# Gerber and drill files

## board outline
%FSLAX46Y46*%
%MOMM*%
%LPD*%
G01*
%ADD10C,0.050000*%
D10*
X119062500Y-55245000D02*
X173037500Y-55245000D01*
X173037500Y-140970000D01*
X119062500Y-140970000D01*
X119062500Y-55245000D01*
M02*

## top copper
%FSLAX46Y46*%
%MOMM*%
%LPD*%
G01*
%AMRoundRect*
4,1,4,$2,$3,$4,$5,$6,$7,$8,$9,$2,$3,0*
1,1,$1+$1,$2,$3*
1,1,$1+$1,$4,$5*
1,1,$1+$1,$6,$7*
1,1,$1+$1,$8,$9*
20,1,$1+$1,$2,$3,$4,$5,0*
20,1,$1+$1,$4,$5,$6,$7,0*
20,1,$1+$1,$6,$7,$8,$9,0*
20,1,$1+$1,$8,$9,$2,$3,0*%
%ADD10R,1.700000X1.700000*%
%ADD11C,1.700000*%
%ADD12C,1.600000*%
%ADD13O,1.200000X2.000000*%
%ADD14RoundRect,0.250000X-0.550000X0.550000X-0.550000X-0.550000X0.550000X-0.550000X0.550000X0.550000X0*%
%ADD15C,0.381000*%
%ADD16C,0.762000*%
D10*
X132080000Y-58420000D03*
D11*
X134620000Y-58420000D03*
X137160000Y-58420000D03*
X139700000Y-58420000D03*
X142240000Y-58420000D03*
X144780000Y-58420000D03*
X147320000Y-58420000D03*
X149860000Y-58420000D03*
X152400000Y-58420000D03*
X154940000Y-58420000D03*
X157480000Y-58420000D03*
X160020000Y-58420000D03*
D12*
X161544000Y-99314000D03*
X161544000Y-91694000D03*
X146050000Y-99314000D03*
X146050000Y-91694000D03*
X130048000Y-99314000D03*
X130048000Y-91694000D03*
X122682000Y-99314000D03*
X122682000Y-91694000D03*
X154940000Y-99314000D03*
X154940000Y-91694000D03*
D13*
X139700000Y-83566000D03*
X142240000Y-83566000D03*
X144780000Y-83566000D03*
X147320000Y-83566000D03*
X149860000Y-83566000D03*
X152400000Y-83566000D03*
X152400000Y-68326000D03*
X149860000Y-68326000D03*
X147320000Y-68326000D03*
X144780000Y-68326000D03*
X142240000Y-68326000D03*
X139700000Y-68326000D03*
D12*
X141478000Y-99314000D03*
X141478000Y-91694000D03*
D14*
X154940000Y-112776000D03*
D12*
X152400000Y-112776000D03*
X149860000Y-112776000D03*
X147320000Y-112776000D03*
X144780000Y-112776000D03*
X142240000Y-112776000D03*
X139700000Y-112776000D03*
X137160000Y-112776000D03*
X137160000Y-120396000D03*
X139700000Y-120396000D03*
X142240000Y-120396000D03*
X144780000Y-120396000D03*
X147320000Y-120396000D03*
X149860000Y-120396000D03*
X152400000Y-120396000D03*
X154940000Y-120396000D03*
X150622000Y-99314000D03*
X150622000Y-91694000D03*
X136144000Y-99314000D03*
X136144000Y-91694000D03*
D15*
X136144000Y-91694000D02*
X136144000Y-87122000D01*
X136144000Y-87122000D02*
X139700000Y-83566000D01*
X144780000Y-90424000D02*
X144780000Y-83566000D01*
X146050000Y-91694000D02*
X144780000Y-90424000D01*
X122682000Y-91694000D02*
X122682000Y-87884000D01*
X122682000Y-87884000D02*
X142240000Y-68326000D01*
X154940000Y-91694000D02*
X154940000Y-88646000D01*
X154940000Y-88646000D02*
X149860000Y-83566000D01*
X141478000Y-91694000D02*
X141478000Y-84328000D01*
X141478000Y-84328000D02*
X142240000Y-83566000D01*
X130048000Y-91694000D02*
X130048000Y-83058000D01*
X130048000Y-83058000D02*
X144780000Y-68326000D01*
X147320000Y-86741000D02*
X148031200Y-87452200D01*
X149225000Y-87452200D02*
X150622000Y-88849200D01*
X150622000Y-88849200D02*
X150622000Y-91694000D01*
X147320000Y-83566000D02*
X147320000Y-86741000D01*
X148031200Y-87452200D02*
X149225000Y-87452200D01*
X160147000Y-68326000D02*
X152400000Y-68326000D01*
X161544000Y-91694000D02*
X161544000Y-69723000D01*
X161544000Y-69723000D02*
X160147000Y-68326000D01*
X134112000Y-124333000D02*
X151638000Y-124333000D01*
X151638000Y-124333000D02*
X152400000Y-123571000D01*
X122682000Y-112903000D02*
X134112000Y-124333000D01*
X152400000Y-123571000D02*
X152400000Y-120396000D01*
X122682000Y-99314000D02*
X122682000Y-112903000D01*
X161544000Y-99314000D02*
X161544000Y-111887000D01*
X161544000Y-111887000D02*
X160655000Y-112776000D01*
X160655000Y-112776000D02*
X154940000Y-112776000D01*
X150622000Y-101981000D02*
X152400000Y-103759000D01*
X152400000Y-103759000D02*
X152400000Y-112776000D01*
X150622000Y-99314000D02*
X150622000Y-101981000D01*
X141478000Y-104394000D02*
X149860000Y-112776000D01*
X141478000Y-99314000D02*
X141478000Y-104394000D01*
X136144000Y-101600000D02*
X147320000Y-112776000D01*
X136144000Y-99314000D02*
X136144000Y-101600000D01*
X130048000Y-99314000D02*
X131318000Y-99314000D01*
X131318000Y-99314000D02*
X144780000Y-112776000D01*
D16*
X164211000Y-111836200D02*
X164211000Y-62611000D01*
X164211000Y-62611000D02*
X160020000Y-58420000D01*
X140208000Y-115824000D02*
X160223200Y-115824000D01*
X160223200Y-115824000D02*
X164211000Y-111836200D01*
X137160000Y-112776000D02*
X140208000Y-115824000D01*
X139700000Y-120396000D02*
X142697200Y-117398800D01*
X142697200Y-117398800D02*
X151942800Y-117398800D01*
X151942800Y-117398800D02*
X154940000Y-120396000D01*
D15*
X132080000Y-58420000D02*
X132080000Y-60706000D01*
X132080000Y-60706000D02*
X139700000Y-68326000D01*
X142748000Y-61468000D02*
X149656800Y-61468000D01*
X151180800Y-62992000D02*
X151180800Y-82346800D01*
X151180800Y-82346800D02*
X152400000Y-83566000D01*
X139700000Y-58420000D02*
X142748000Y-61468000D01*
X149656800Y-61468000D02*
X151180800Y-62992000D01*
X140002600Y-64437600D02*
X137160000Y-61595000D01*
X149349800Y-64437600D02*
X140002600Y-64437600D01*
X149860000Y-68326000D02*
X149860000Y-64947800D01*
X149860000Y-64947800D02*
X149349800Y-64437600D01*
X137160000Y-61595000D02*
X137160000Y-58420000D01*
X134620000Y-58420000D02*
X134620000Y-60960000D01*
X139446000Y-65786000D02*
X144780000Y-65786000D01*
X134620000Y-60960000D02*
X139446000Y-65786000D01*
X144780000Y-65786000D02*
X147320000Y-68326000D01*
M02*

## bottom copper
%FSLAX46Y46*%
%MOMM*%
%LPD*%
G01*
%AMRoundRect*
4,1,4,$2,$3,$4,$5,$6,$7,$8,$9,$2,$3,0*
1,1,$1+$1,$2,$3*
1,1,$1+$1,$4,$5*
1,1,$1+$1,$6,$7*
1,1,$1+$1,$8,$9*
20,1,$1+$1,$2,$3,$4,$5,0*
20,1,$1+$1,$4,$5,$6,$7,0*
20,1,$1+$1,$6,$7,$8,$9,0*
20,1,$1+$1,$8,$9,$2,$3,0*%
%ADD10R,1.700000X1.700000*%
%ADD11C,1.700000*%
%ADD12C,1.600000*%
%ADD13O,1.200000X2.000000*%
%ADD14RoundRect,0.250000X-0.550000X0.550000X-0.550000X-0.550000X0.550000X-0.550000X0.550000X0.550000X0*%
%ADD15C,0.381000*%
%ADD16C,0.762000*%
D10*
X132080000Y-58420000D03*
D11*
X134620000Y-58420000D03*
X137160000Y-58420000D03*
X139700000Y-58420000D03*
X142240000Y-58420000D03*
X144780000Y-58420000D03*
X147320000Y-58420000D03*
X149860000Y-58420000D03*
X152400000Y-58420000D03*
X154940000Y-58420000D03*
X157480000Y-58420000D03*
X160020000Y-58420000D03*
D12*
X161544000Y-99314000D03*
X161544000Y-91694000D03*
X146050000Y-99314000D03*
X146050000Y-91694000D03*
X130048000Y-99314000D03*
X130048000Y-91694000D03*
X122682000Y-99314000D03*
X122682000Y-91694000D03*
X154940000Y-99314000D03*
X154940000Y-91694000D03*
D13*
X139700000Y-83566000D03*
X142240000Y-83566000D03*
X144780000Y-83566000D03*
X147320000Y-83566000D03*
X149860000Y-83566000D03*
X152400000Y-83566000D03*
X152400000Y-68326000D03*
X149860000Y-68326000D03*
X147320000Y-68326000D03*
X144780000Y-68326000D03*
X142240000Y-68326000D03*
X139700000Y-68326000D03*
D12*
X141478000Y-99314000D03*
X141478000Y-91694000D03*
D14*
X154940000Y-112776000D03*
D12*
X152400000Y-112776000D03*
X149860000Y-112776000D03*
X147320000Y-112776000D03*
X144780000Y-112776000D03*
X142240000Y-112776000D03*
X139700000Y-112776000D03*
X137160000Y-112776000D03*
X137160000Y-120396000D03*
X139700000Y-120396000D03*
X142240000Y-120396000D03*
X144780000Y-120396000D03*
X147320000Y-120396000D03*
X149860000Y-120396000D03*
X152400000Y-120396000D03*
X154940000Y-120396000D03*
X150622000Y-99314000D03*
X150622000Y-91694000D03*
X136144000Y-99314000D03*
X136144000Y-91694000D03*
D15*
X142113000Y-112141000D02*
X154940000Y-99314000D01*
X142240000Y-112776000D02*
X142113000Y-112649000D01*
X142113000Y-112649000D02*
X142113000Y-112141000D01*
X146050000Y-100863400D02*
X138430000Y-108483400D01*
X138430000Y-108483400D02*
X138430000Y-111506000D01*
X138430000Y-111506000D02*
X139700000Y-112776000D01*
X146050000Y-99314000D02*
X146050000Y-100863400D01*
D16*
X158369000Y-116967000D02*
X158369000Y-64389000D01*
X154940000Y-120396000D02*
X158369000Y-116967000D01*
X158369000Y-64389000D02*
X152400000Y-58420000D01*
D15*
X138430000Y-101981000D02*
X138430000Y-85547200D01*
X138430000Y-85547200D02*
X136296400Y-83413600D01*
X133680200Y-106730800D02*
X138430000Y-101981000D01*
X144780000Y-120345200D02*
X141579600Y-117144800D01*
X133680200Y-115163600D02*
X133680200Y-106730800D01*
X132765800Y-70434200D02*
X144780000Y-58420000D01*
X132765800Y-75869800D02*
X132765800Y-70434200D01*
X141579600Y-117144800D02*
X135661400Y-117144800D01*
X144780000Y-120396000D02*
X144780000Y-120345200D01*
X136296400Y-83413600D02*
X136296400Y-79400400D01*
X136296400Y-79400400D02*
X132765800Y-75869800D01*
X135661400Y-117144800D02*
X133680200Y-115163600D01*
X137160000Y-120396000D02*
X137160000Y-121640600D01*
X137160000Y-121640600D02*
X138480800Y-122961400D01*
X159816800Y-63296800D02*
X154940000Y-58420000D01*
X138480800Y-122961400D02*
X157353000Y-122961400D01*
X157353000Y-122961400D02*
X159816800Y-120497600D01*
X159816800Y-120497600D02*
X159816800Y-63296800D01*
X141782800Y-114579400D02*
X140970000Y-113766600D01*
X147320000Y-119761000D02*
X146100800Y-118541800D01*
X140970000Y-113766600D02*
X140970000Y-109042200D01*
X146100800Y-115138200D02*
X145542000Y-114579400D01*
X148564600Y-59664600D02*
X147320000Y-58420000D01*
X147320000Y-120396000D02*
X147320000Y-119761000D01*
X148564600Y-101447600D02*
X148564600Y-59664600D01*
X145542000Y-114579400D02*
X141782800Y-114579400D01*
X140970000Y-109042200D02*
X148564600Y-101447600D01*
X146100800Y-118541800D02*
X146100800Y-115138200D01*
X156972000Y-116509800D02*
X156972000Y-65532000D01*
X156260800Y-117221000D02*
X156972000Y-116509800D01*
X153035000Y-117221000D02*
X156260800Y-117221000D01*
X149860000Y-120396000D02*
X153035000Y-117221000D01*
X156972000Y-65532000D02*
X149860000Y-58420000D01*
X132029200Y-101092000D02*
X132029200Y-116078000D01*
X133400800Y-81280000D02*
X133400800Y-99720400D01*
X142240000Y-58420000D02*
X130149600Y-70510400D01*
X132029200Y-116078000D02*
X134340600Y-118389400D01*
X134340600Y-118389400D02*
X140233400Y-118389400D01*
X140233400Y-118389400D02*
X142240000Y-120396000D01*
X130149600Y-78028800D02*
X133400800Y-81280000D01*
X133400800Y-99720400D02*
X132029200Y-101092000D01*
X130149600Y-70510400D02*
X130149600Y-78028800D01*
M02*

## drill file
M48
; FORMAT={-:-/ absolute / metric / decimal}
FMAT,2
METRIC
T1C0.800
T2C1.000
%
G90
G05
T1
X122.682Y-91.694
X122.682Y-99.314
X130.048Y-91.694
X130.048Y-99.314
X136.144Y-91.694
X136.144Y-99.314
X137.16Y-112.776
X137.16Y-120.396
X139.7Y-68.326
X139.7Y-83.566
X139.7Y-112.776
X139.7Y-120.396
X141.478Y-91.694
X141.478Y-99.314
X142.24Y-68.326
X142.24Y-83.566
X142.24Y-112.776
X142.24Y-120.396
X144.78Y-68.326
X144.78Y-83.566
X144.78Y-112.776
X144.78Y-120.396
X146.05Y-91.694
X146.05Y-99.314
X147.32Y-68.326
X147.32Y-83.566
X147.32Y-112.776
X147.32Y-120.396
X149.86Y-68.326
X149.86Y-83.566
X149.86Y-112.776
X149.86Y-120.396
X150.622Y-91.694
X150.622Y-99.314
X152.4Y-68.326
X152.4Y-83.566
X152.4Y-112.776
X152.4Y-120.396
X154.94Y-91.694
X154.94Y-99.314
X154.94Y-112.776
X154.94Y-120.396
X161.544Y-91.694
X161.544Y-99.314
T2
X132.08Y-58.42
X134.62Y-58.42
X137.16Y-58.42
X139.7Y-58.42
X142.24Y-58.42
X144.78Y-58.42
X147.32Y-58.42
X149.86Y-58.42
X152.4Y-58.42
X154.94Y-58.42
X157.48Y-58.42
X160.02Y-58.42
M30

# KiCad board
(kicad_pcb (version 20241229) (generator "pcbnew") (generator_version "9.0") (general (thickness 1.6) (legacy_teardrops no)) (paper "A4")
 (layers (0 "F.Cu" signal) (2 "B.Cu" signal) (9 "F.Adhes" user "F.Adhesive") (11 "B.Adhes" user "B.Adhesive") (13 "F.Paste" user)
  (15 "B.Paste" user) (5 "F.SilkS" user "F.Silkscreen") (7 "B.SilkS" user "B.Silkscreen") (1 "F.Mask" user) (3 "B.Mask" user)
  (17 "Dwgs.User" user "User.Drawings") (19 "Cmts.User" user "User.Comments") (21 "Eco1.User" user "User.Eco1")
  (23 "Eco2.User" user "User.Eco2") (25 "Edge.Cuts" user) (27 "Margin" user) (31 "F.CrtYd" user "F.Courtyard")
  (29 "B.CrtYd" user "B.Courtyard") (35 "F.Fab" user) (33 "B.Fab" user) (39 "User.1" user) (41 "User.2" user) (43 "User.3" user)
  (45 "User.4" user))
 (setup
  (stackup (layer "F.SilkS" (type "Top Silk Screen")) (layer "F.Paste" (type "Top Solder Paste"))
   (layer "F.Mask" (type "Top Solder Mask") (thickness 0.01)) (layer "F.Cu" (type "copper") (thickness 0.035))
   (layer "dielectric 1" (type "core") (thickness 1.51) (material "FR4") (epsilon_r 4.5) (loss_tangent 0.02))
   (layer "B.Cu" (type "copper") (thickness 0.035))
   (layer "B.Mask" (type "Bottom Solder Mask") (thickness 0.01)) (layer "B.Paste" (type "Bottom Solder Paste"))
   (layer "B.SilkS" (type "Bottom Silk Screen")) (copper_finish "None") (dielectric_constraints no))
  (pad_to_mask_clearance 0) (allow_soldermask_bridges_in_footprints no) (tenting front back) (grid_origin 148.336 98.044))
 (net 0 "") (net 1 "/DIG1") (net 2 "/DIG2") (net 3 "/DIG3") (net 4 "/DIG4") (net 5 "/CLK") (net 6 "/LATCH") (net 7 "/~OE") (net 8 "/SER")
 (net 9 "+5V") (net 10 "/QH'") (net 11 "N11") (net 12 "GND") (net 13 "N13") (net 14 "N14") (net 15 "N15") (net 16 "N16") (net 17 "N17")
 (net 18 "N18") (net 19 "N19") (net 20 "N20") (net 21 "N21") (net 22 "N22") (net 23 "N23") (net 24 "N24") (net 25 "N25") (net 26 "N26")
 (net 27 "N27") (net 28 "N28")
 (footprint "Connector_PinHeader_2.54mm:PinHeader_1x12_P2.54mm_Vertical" (layer "F.Cu") (at 132.08 58.42 90)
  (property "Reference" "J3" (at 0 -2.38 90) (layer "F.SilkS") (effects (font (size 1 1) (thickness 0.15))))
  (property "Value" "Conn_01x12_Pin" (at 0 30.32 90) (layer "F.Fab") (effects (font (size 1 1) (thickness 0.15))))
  (pad "1" thru_hole rect (at 0 0 90) (size 1.7 1.7) (drill 1) (layers "*.Cu" "*.Mask") (remove_unused_layers no) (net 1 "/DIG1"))
  (pad "2" thru_hole circle (at 0 2.54 90) (size 1.7 1.7) (drill 1) (layers "*.Cu" "*.Mask") (remove_unused_layers no) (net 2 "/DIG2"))
  (pad "3" thru_hole circle (at 0 5.08 90) (size 1.7 1.7) (drill 1) (layers "*.Cu" "*.Mask") (remove_unused_layers no) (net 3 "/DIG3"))
  (pad "4" thru_hole circle (at 0 7.62 90) (size 1.7 1.7) (drill 1) (layers "*.Cu" "*.Mask") (remove_unused_layers no) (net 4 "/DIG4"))
  (pad "5" thru_hole circle (at 0 10.16 90) (size 1.7 1.7) (drill 1) (layers "*.Cu" "*.Mask") (remove_unused_layers no) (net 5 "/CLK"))
  (pad "6" thru_hole circle (at 0 12.7 90) (size 1.7 1.7) (drill 1) (layers "*.Cu" "*.Mask") (remove_unused_layers no) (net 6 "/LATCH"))
  (pad "7" thru_hole circle (at 0 15.24 90) (size 1.7 1.7) (drill 1) (layers "*.Cu" "*.Mask") (remove_unused_layers no) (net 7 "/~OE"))
  (pad "8" thru_hole circle (at 0 17.78 90) (size 1.7 1.7) (drill 1) (layers "*.Cu" "*.Mask") (remove_unused_layers no) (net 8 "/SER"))
  (pad "9" thru_hole circle (at 0 20.32 90) (size 1.7 1.7) (drill 1) (layers "*.Cu" "*.Mask") (remove_unused_layers no) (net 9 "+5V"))
  (pad "10" thru_hole circle (at 0 22.86 90) (size 1.7 1.7) (drill 1) (layers "*.Cu" "*.Mask") (remove_unused_layers no) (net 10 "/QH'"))
  (pad "11" thru_hole circle (at 0 25.4 90) (size 1.7 1.7) (drill 1) (layers "*.Cu" "*.Mask") (remove_unused_layers no) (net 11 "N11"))
  (pad "12" thru_hole circle (at 0 27.94 90) (size 1.7 1.7) (drill 1) (layers "*.Cu" "*.Mask") (remove_unused_layers no) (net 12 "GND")))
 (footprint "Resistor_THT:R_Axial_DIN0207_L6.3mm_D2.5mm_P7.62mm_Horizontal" (layer "F.Cu") (at 161.544 99.314 90)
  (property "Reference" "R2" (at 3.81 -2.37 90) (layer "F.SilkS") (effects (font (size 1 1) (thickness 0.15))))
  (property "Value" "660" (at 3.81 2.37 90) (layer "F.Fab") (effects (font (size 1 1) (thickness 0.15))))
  (pad "1" thru_hole circle (at 0 0 90) (size 1.6 1.6) (drill 0.8) (layers "*.Cu" "*.Mask") (remove_unused_layers no) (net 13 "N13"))
  (pad "2" thru_hole circle (at 7.62 0 90) (size 1.6 1.6) (drill 0.8) (layers "*.Cu" "*.Mask") (remove_unused_layers no) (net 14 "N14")))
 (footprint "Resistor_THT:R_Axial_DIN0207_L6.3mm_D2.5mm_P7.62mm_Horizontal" (layer "F.Cu") (at 146.05 99.314 90)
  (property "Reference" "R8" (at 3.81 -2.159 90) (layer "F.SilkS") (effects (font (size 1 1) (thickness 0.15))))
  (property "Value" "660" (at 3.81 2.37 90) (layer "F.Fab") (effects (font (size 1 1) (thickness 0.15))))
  (pad "1" thru_hole circle (at 0 0 90) (size 1.6 1.6) (drill 0.8) (layers "*.Cu" "*.Mask") (remove_unused_layers no) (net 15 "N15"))
  (pad "2" thru_hole circle (at 7.62 0 90) (size 1.6 1.6) (drill 0.8) (layers "*.Cu" "*.Mask") (remove_unused_layers no) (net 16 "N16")))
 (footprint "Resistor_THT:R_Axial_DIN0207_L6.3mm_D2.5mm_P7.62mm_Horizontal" (layer "F.Cu") (at 130.048 99.314 90)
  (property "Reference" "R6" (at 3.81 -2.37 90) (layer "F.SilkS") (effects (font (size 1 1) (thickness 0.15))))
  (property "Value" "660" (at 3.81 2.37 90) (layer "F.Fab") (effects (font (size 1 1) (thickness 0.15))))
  (pad "1" thru_hole circle (at 0 0 90) (size 1.6 1.6) (drill 0.8) (layers "*.Cu" "*.Mask") (remove_unused_layers no) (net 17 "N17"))
  (pad "2" thru_hole circle (at 7.62 0 90) (size 1.6 1.6) (drill 0.8) (layers "*.Cu" "*.Mask") (remove_unused_layers no) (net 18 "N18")))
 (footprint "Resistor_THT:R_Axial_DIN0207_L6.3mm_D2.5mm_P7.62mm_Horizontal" (layer "F.Cu") (at 122.682 99.314 90)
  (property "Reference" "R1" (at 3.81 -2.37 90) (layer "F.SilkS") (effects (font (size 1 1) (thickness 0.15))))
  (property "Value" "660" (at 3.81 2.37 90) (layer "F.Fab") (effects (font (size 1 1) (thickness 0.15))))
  (pad "1" thru_hole circle (at 0 0 90) (size 1.6 1.6) (drill 0.8) (layers "*.Cu" "*.Mask") (remove_unused_layers no) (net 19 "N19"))
  (pad "2" thru_hole circle (at 7.62 0 90) (size 1.6 1.6) (drill 0.8) (layers "*.Cu" "*.Mask") (remove_unused_layers no) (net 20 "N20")))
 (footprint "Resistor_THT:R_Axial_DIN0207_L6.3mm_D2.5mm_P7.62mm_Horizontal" (layer "F.Cu") (at 154.94 99.314 90)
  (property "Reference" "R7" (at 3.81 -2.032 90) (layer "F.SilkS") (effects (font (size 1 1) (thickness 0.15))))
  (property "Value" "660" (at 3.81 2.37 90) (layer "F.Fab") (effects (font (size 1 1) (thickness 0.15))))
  (pad "1" thru_hole circle (at 0 0 90) (size 1.6 1.6) (drill 0.8) (layers "*.Cu" "*.Mask") (remove_unused_layers no) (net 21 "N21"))
  (pad "2" thru_hole circle (at 7.62 0 90) (size 1.6 1.6) (drill 0.8) (layers "*.Cu" "*.Mask") (remove_unused_layers no) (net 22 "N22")))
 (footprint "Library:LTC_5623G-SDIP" (layer "F.Cu") (at 146.05 75.946)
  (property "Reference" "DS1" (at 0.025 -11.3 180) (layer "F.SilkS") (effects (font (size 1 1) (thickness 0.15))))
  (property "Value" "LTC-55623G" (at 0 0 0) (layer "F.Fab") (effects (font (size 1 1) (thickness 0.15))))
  (pad "1" thru_hole oval (at -6.35 7.62) (size 1.2 2) (drill 0.8) (layers "*.Cu" "*.Mask") (remove_unused_layers no) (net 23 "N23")
   (thermal_bridge_angle 45))
  (pad "2" thru_hole oval (at -3.81 7.62) (size 1.2 2) (drill 0.8) (layers "*.Cu" "*.Mask") (remove_unused_layers no) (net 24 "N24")
   (thermal_bridge_angle 45))
  (pad "3" thru_hole oval (at -1.27 7.62) (size 1.2 2) (drill 0.8) (layers "*.Cu" "*.Mask") (remove_unused_layers no) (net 16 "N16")
   (thermal_bridge_angle 45))
  (pad "4" thru_hole oval (at 1.27 7.62) (size 1.2 2) (drill 0.8) (layers "*.Cu" "*.Mask") (remove_unused_layers no) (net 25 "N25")
   (thermal_bridge_angle 45))
  (pad "5" thru_hole oval (at 3.81 7.62) (size 1.2 2) (drill 0.8) (layers "*.Cu" "*.Mask") (remove_unused_layers no) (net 22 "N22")
   (thermal_bridge_angle 45))
  (pad "6" thru_hole oval (at 6.35 7.62) (size 1.2 2) (drill 0.8) (layers "*.Cu" "*.Mask") (remove_unused_layers no) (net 4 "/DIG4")
   (thermal_bridge_angle 45))
  (pad "7" thru_hole oval (at 6.35 -7.62) (size 1.2 2) (drill 0.8) (layers "*.Cu" "*.Mask") (remove_unused_layers no) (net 14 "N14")
   (thermal_bridge_angle 45))
  (pad "8" thru_hole oval (at 3.81 -7.62) (size 1.2 2) (drill 0.8) (layers "*.Cu" "*.Mask") (remove_unused_layers no) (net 3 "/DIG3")
   (thermal_bridge_angle 45))
  (pad "9" thru_hole oval (at 1.27 -7.62) (size 1.2 2) (drill 0.8) (layers "*.Cu" "*.Mask") (remove_unused_layers no) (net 2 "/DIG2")
   (thermal_bridge_angle 45))
  (pad "10" thru_hole oval (at -1.27 -7.62) (size 1.2 2) (drill 0.8) (layers "*.Cu" "*.Mask") (remove_unused_layers no) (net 18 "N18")
   (thermal_bridge_angle 45))
  (pad "11" thru_hole oval (at -3.81 -7.62) (size 1.2 2) (drill 0.8) (layers "*.Cu" "*.Mask") (remove_unused_layers no) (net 20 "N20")
   (thermal_bridge_angle 45))
  (pad "12" thru_hole oval (at -6.35 -7.62) (size 1.2 2) (drill 0.8) (layers "*.Cu" "*.Mask") (remove_unused_layers no) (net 1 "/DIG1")
   (thermal_bridge_angle 45)))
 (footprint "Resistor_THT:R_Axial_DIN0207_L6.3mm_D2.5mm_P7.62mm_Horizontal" (layer "F.Cu") (at 141.478 99.314 90)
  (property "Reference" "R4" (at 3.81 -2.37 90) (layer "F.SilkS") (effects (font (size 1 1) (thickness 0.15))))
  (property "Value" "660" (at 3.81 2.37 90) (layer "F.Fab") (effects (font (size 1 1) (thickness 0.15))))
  (pad "1" thru_hole circle (at 0 0 90) (size 1.6 1.6) (drill 0.8) (layers "*.Cu" "*.Mask") (remove_unused_layers no) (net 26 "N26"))
  (pad "2" thru_hole circle (at 7.62 0 90) (size 1.6 1.6) (drill 0.8) (layers "*.Cu" "*.Mask") (remove_unused_layers no) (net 24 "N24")))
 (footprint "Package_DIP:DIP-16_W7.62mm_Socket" (layer "F.Cu") (at 154.94 112.776 -90)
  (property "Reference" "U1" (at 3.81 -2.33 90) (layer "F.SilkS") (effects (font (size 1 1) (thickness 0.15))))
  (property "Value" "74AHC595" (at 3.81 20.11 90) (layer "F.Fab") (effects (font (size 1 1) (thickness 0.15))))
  (pad "1" thru_hole roundrect (at 0 0 270) (size 1.6 1.6) (drill 0.8) (layers "*.Cu" "*.Mask") (remove_unused_layers no)
   (roundrect_rratio 0.15625) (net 13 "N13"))
  (pad "2" thru_hole circle (at 0 2.54 270) (size 1.6 1.6) (drill 0.8) (layers "*.Cu" "*.Mask") (remove_unused_layers no) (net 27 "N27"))
  (pad "3" thru_hole circle (at 0 5.08 270) (size 1.6 1.6) (drill 0.8) (layers "*.Cu" "*.Mask") (remove_unused_layers no) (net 26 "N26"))
  (pad "4" thru_hole circle (at 0 7.62 270) (size 1.6 1.6) (drill 0.8) (layers "*.Cu" "*.Mask") (remove_unused_layers no) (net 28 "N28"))
  (pad "5" thru_hole circle (at 0 10.16 270) (size 1.6 1.6) (drill 0.8) (layers "*.Cu" "*.Mask") (remove_unused_layers no) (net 17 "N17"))
  (pad "6" thru_hole circle (at 0 12.7 270) (size 1.6 1.6) (drill 0.8) (layers "*.Cu" "*.Mask") (remove_unused_layers no) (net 21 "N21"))
  (pad "7" thru_hole circle (at 0 15.24 270) (size 1.6 1.6) (drill 0.8) (layers "*.Cu" "*.Mask") (remove_unused_layers no) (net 15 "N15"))
  (pad "8" thru_hole circle (at 0 17.78 270) (size 1.6 1.6) (drill 0.8) (layers "*.Cu" "*.Mask") (remove_unused_layers no) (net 12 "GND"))
  (pad "9" thru_hole circle (at 7.62 17.78 270) (size 1.6 1.6) (drill 0.8) (layers "*.Cu" "*.Mask") (remove_unused_layers no)
   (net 10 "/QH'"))
  (pad "10" thru_hole circle (at 7.62 15.24 270) (size 1.6 1.6) (drill 0.8) (layers "*.Cu" "*.Mask") (remove_unused_layers no) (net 9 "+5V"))
  (pad "11" thru_hole circle (at 7.62 12.7 270) (size 1.6 1.6) (drill 0.8) (layers "*.Cu" "*.Mask") (remove_unused_layers no) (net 5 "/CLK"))
  (pad "12" thru_hole circle (at 7.62 10.16 270) (size 1.6 1.6) (drill 0.8) (layers "*.Cu" "*.Mask") (remove_unused_layers no)
   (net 6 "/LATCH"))
  (pad "13" thru_hole circle (at 7.62 7.62 270) (size 1.6 1.6) (drill 0.8) (layers "*.Cu" "*.Mask") (remove_unused_layers no) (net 7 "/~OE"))
  (pad "14" thru_hole circle (at 7.62 5.08 270) (size 1.6 1.6) (drill 0.8) (layers "*.Cu" "*.Mask") (remove_unused_layers no) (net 8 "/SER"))
  (pad "15" thru_hole circle (at 7.62 2.54 270) (size 1.6 1.6) (drill 0.8) (layers "*.Cu" "*.Mask") (remove_unused_layers no) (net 19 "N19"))
  (pad "16" thru_hole circle (at 7.62 0 270) (size 1.6 1.6) (drill 0.8) (layers "*.Cu" "*.Mask") (remove_unused_layers no) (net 9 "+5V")))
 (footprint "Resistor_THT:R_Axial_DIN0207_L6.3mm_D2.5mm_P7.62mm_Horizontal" (layer "F.Cu") (at 150.622 99.314 90)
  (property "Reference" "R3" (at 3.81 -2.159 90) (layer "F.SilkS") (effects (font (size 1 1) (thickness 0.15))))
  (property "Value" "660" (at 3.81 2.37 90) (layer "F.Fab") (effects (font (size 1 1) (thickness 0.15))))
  (pad "1" thru_hole circle (at 0 0 90) (size 1.6 1.6) (drill 0.8) (layers "*.Cu" "*.Mask") (remove_unused_layers no) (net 27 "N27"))
  (pad "2" thru_hole circle (at 7.62 0 90) (size 1.6 1.6) (drill 0.8) (layers "*.Cu" "*.Mask") (remove_unused_layers no) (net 25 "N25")))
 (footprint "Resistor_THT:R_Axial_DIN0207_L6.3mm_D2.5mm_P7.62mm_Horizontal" (layer "F.Cu") (at 136.144 99.314 90)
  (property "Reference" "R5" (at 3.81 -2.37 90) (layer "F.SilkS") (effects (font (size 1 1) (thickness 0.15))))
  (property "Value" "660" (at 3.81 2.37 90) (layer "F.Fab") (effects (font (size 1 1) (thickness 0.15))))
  (pad "1" thru_hole circle (at 0 0 90) (size 1.6 1.6) (drill 0.8) (layers "*.Cu" "*.Mask") (remove_unused_layers no) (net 28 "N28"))
  (pad "2" thru_hole circle (at 7.62 0 90) (size 1.6 1.6) (drill 0.8) (layers "*.Cu" "*.Mask") (remove_unused_layers no) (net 23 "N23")))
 (gr_rect (start 119.0625 55.245) (end 173.0375 140.97) (stroke (width 0.05) (type solid)) (fill no) (layer "Edge.Cuts"))
 (segment (start 136.144 91.694) (end 136.144 87.122) (width 0.381) (layer "F.Cu") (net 23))
 (segment (start 136.144 87.122) (end 139.7 83.566) (width 0.381) (layer "F.Cu") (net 23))
 (segment (start 144.78 90.424) (end 144.78 83.566) (width 0.381) (layer "F.Cu") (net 16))
 (segment (start 146.05 91.694) (end 144.78 90.424) (width 0.381) (layer "F.Cu") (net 16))
 (segment (start 122.682 91.694) (end 122.682 87.884) (width 0.381) (layer "F.Cu") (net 20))
 (segment (start 122.682 87.884) (end 142.24 68.326) (width 0.381) (layer "F.Cu") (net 20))
 (segment (start 154.94 91.694) (end 154.94 88.646) (width 0.381) (layer "F.Cu") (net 22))
 (segment (start 154.94 88.646) (end 149.86 83.566) (width 0.381) (layer "F.Cu") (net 22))
 (segment (start 141.478 91.694) (end 141.478 84.328) (width 0.381) (layer "F.Cu") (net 24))
 (segment (start 141.478 84.328) (end 142.24 83.566) (width 0.381) (layer "F.Cu") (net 24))
 (segment (start 130.048 91.694) (end 130.048 83.058) (width 0.381) (layer "F.Cu") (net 18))
 (segment (start 130.048 83.058) (end 144.78 68.326) (width 0.381) (layer "F.Cu") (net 18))
 (segment (start 147.32 86.741) (end 148.0312 87.4522) (width 0.381) (layer "F.Cu") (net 25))
 (segment (start 149.225 87.4522) (end 150.622 88.8492) (width 0.381) (layer "F.Cu") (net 25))
 (segment (start 150.622 88.8492) (end 150.622 91.694) (width 0.381) (layer "F.Cu") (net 25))
 (segment (start 147.32 83.566) (end 147.32 86.741) (width 0.381) (layer "F.Cu") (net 25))
 (segment (start 148.0312 87.4522) (end 149.225 87.4522) (width 0.381) (layer "F.Cu") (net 25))
 (segment (start 160.147 68.326) (end 152.4 68.326) (width 0.381) (layer "F.Cu") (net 14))
 (segment (start 161.544 91.694) (end 161.544 69.723) (width 0.381) (layer "F.Cu") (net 14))
 (segment (start 161.544 69.723) (end 160.147 68.326) (width 0.381) (layer "F.Cu") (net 14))
 (segment (start 134.112 124.333) (end 151.638 124.333) (width 0.381) (layer "F.Cu") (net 19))
 (segment (start 151.638 124.333) (end 152.4 123.571) (width 0.381) (layer "F.Cu") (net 19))
 (segment (start 122.682 112.903) (end 134.112 124.333) (width 0.381) (layer "F.Cu") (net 19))
 (segment (start 152.4 123.571) (end 152.4 120.396) (width 0.381) (layer "F.Cu") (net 19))
 (segment (start 122.682 99.314) (end 122.682 112.903) (width 0.381) (layer "F.Cu") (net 19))
 (segment (start 161.544 99.314) (end 161.544 111.887) (width 0.381) (layer "F.Cu") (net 13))
 (segment (start 161.544 111.887) (end 160.655 112.776) (width 0.381) (layer "F.Cu") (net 13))
 (segment (start 160.655 112.776) (end 154.94 112.776) (width 0.381) (layer "F.Cu") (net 13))
 (segment (start 150.622 101.981) (end 152.4 103.759) (width 0.381) (layer "F.Cu") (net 27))
 (segment (start 152.4 103.759) (end 152.4 112.776) (width 0.381) (layer "F.Cu") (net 27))
 (segment (start 150.622 99.314) (end 150.622 101.981) (width 0.381) (layer "F.Cu") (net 27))
 (segment (start 141.478 104.394) (end 149.86 112.776) (width 0.381) (layer "F.Cu") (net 26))
 (segment (start 141.478 99.314) (end 141.478 104.394) (width 0.381) (layer "F.Cu") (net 26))
 (segment (start 136.144 101.6) (end 147.32 112.776) (width 0.381) (layer "F.Cu") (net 28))
 (segment (start 136.144 99.314) (end 136.144 101.6) (width 0.381) (layer "F.Cu") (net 28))
 (segment (start 130.048 99.314) (end 131.318 99.314) (width 0.381) (layer "F.Cu") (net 17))
 (segment (start 131.318 99.314) (end 144.78 112.776) (width 0.381) (layer "F.Cu") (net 17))
 (segment (start 142.113 112.141) (end 154.94 99.314) (width 0.381) (layer "B.Cu") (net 21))
 (segment (start 142.24 112.776) (end 142.113 112.649) (width 0.381) (layer "B.Cu") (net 21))
 (segment (start 142.113 112.649) (end 142.113 112.141) (width 0.381) (layer "B.Cu") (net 21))
 (segment (start 146.05 100.8634) (end 138.43 108.4834) (width 0.381) (layer "B.Cu") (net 15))
 (segment (start 138.43 108.4834) (end 138.43 111.506) (width 0.381) (layer "B.Cu") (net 15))
 (segment (start 138.43 111.506) (end 139.7 112.776) (width 0.381) (layer "B.Cu") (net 15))
 (segment (start 146.05 99.314) (end 146.05 100.8634) (width 0.381) (layer "B.Cu") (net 15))
 (segment (start 164.211 111.8362) (end 164.211 62.611) (width 0.762) (layer "F.Cu") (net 12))
 (segment (start 164.211 62.611) (end 160.02 58.42) (width 0.762) (layer "F.Cu") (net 12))
 (segment (start 140.208 115.824) (end 160.2232 115.824) (width 0.762) (layer "F.Cu") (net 12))
 (segment (start 160.2232 115.824) (end 164.211 111.8362) (width 0.762) (layer "F.Cu") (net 12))
 (segment (start 137.16 112.776) (end 140.208 115.824) (width 0.762) (layer "F.Cu") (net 12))
 (segment (start 139.7 120.396) (end 142.6972 117.3988) (width 0.762) (layer "F.Cu") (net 9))
 (segment (start 142.6972 117.3988) (end 151.9428 117.3988) (width 0.762) (layer "F.Cu") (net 9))
 (segment (start 151.9428 117.3988) (end 154.94 120.396) (width 0.762) (layer "F.Cu") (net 9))
 (segment (start 158.369 116.967) (end 158.369 64.389) (width 0.762) (layer "B.Cu") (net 9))
 (segment (start 154.94 120.396) (end 158.369 116.967) (width 0.762) (layer "B.Cu") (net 9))
 (segment (start 158.369 64.389) (end 152.4 58.42) (width 0.762) (layer "B.Cu") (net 9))
 (segment (start 132.08 58.42) (end 132.08 60.706) (width 0.381) (layer "F.Cu") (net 1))
 (segment (start 132.08 60.706) (end 139.7 68.326) (width 0.381) (layer "F.Cu") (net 1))
 (segment (start 142.748 61.468) (end 149.6568 61.468) (width 0.381) (layer "F.Cu") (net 4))
 (segment (start 151.1808 62.992) (end 151.1808 82.3468) (width 0.381) (layer "F.Cu") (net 4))
 (segment (start 151.1808 82.3468) (end 152.4 83.566) (width 0.381) (layer "F.Cu") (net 4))
 (segment (start 139.7 58.42) (end 142.748 61.468) (width 0.381) (layer "F.Cu") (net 4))
 (segment (start 149.6568 61.468) (end 151.1808 62.992) (width 0.381) (layer "F.Cu") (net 4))
 (segment (start 140.0026 64.4376) (end 137.16 61.595) (width 0.381) (layer "F.Cu") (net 3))
 (segment (start 149.3498 64.4376) (end 140.0026 64.4376) (width 0.381) (layer "F.Cu") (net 3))
 (segment (start 149.86 68.326) (end 149.86 64.9478) (width 0.381) (layer "F.Cu") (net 3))
 (segment (start 149.86 64.9478) (end 149.3498 64.4376) (width 0.381) (layer "F.Cu") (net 3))
 (segment (start 137.16 61.595) (end 137.16 58.42) (width 0.381) (layer "F.Cu") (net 3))
 (segment (start 134.62 58.42) (end 134.62 60.96) (width 0.381) (layer "F.Cu") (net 2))
 (segment (start 139.446 65.786) (end 144.78 65.786) (width 0.381) (layer "F.Cu") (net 2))
 (segment (start 134.62 60.96) (end 139.446 65.786) (width 0.381) (layer "F.Cu") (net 2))
 (segment (start 144.78 65.786) (end 147.32 68.326) (width 0.381) (layer "F.Cu") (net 2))
 (segment (start 138.43 101.981) (end 138.43 85.5472) (width 0.381) (layer "B.Cu") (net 6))
 (segment (start 138.43 85.5472) (end 136.2964 83.4136) (width 0.381) (layer "B.Cu") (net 6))
 (segment (start 133.6802 106.7308) (end 138.43 101.981) (width 0.381) (layer "B.Cu") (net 6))
 (segment (start 144.78 120.3452) (end 141.5796 117.1448) (width 0.381) (layer "B.Cu") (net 6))
 (segment (start 133.6802 115.1636) (end 133.6802 106.7308) (width 0.381) (layer "B.Cu") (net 6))
 (segment (start 132.7658 70.4342) (end 144.78 58.42) (width 0.381) (layer "B.Cu") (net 6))
 (segment (start 132.7658 75.8698) (end 132.7658 70.4342) (width 0.381) (layer "B.Cu") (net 6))
 (segment (start 141.5796 117.1448) (end 135.6614 117.1448) (width 0.381) (layer "B.Cu") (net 6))
 (segment (start 144.78 120.396) (end 144.78 120.3452) (width 0.381) (layer "B.Cu") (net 6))
 (segment (start 136.2964 83.4136) (end 136.2964 79.4004) (width 0.381) (layer "B.Cu") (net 6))
 (segment (start 136.2964 79.4004) (end 132.7658 75.8698) (width 0.381) (layer "B.Cu") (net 6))
 (segment (start 135.6614 117.1448) (end 133.6802 115.1636) (width 0.381) (layer "B.Cu") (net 6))
 (segment (start 137.16 120.396) (end 137.16 121.6406) (width 0.381) (layer "B.Cu") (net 10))
 (segment (start 137.16 121.6406) (end 138.4808 122.9614) (width 0.381) (layer "B.Cu") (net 10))
 (segment (start 159.8168 63.2968) (end 154.94 58.42) (width 0.381) (layer "B.Cu") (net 10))
 (segment (start 138.4808 122.9614) (end 157.353 122.9614) (width 0.381) (layer "B.Cu") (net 10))
 (segment (start 157.353 122.9614) (end 159.8168 120.4976) (width 0.381) (layer "B.Cu") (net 10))
 (segment (start 159.8168 120.4976) (end 159.8168 63.2968) (width 0.381) (layer "B.Cu") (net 10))
 (segment (start 141.7828 114.5794) (end 140.97 113.7666) (width 0.381) (layer "B.Cu") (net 7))
 (segment (start 147.32 119.761) (end 146.1008 118.5418) (width 0.381) (layer "B.Cu") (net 7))
 (segment (start 140.97 113.7666) (end 140.97 109.0422) (width 0.381) (layer "B.Cu") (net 7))
 (segment (start 146.1008 115.1382) (end 145.542 114.5794) (width 0.381) (layer "B.Cu") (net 7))
 (segment (start 148.5646 59.6646) (end 147.32 58.42) (width 0.381) (layer "B.Cu") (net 7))
 (segment (start 147.32 120.396) (end 147.32 119.761) (width 0.381) (layer "B.Cu") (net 7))
 (segment (start 148.5646 101.4476) (end 148.5646 59.6646) (width 0.381) (layer "B.Cu") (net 7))
 (segment (start 145.542 114.5794) (end 141.7828 114.5794) (width 0.381) (layer "B.Cu") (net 7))
 (segment (start 140.97 109.0422) (end 148.5646 101.4476) (width 0.381) (layer "B.Cu") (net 7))
 (segment (start 146.1008 118.5418) (end 146.1008 115.1382) (width 0.381) (layer "B.Cu") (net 7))
 (segment (start 156.972 116.5098) (end 156.972 65.532) (width 0.381) (layer "B.Cu") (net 8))
 (segment (start 156.2608 117.221) (end 156.972 116.5098) (width 0.381) (layer "B.Cu") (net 8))
 (segment (start 153.035 117.221) (end 156.2608 117.221) (width 0.381) (layer "B.Cu") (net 8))
 (segment (start 149.86 120.396) (end 153.035 117.221) (width 0.381) (layer "B.Cu") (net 8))
 (segment (start 156.972 65.532) (end 149.86 58.42) (width 0.381) (layer "B.Cu") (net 8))
 (segment (start 132.0292 101.092) (end 132.0292 116.078) (width 0.381) (layer "B.Cu") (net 5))
 (segment (start 133.4008 81.28) (end 133.4008 99.7204) (width 0.381) (layer "B.Cu") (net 5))
 (segment (start 142.24 58.42) (end 130.1496 70.5104) (width 0.381) (layer "B.Cu") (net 5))
 (segment (start 132.0292 116.078) (end 134.3406 118.3894) (width 0.381) (layer "B.Cu") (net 5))
 (segment (start 134.3406 118.3894) (end 140.2334 118.3894) (width 0.381) (layer "B.Cu") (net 5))
 (segment (start 140.2334 118.3894) (end 142.24 120.396) (width 0.381) (layer "B.Cu") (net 5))
 (segment (start 130.1496 78.0288) (end 133.4008 81.28) (width 0.381) (layer "B.Cu") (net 5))
 (segment (start 133.4008 99.7204) (end 132.0292 101.092) (width 0.381) (layer "B.Cu") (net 5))
 (segment (start 130.1496 70.5104) (end 130.1496 78.0288) (width 0.381) (layer "B.Cu") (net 5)))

